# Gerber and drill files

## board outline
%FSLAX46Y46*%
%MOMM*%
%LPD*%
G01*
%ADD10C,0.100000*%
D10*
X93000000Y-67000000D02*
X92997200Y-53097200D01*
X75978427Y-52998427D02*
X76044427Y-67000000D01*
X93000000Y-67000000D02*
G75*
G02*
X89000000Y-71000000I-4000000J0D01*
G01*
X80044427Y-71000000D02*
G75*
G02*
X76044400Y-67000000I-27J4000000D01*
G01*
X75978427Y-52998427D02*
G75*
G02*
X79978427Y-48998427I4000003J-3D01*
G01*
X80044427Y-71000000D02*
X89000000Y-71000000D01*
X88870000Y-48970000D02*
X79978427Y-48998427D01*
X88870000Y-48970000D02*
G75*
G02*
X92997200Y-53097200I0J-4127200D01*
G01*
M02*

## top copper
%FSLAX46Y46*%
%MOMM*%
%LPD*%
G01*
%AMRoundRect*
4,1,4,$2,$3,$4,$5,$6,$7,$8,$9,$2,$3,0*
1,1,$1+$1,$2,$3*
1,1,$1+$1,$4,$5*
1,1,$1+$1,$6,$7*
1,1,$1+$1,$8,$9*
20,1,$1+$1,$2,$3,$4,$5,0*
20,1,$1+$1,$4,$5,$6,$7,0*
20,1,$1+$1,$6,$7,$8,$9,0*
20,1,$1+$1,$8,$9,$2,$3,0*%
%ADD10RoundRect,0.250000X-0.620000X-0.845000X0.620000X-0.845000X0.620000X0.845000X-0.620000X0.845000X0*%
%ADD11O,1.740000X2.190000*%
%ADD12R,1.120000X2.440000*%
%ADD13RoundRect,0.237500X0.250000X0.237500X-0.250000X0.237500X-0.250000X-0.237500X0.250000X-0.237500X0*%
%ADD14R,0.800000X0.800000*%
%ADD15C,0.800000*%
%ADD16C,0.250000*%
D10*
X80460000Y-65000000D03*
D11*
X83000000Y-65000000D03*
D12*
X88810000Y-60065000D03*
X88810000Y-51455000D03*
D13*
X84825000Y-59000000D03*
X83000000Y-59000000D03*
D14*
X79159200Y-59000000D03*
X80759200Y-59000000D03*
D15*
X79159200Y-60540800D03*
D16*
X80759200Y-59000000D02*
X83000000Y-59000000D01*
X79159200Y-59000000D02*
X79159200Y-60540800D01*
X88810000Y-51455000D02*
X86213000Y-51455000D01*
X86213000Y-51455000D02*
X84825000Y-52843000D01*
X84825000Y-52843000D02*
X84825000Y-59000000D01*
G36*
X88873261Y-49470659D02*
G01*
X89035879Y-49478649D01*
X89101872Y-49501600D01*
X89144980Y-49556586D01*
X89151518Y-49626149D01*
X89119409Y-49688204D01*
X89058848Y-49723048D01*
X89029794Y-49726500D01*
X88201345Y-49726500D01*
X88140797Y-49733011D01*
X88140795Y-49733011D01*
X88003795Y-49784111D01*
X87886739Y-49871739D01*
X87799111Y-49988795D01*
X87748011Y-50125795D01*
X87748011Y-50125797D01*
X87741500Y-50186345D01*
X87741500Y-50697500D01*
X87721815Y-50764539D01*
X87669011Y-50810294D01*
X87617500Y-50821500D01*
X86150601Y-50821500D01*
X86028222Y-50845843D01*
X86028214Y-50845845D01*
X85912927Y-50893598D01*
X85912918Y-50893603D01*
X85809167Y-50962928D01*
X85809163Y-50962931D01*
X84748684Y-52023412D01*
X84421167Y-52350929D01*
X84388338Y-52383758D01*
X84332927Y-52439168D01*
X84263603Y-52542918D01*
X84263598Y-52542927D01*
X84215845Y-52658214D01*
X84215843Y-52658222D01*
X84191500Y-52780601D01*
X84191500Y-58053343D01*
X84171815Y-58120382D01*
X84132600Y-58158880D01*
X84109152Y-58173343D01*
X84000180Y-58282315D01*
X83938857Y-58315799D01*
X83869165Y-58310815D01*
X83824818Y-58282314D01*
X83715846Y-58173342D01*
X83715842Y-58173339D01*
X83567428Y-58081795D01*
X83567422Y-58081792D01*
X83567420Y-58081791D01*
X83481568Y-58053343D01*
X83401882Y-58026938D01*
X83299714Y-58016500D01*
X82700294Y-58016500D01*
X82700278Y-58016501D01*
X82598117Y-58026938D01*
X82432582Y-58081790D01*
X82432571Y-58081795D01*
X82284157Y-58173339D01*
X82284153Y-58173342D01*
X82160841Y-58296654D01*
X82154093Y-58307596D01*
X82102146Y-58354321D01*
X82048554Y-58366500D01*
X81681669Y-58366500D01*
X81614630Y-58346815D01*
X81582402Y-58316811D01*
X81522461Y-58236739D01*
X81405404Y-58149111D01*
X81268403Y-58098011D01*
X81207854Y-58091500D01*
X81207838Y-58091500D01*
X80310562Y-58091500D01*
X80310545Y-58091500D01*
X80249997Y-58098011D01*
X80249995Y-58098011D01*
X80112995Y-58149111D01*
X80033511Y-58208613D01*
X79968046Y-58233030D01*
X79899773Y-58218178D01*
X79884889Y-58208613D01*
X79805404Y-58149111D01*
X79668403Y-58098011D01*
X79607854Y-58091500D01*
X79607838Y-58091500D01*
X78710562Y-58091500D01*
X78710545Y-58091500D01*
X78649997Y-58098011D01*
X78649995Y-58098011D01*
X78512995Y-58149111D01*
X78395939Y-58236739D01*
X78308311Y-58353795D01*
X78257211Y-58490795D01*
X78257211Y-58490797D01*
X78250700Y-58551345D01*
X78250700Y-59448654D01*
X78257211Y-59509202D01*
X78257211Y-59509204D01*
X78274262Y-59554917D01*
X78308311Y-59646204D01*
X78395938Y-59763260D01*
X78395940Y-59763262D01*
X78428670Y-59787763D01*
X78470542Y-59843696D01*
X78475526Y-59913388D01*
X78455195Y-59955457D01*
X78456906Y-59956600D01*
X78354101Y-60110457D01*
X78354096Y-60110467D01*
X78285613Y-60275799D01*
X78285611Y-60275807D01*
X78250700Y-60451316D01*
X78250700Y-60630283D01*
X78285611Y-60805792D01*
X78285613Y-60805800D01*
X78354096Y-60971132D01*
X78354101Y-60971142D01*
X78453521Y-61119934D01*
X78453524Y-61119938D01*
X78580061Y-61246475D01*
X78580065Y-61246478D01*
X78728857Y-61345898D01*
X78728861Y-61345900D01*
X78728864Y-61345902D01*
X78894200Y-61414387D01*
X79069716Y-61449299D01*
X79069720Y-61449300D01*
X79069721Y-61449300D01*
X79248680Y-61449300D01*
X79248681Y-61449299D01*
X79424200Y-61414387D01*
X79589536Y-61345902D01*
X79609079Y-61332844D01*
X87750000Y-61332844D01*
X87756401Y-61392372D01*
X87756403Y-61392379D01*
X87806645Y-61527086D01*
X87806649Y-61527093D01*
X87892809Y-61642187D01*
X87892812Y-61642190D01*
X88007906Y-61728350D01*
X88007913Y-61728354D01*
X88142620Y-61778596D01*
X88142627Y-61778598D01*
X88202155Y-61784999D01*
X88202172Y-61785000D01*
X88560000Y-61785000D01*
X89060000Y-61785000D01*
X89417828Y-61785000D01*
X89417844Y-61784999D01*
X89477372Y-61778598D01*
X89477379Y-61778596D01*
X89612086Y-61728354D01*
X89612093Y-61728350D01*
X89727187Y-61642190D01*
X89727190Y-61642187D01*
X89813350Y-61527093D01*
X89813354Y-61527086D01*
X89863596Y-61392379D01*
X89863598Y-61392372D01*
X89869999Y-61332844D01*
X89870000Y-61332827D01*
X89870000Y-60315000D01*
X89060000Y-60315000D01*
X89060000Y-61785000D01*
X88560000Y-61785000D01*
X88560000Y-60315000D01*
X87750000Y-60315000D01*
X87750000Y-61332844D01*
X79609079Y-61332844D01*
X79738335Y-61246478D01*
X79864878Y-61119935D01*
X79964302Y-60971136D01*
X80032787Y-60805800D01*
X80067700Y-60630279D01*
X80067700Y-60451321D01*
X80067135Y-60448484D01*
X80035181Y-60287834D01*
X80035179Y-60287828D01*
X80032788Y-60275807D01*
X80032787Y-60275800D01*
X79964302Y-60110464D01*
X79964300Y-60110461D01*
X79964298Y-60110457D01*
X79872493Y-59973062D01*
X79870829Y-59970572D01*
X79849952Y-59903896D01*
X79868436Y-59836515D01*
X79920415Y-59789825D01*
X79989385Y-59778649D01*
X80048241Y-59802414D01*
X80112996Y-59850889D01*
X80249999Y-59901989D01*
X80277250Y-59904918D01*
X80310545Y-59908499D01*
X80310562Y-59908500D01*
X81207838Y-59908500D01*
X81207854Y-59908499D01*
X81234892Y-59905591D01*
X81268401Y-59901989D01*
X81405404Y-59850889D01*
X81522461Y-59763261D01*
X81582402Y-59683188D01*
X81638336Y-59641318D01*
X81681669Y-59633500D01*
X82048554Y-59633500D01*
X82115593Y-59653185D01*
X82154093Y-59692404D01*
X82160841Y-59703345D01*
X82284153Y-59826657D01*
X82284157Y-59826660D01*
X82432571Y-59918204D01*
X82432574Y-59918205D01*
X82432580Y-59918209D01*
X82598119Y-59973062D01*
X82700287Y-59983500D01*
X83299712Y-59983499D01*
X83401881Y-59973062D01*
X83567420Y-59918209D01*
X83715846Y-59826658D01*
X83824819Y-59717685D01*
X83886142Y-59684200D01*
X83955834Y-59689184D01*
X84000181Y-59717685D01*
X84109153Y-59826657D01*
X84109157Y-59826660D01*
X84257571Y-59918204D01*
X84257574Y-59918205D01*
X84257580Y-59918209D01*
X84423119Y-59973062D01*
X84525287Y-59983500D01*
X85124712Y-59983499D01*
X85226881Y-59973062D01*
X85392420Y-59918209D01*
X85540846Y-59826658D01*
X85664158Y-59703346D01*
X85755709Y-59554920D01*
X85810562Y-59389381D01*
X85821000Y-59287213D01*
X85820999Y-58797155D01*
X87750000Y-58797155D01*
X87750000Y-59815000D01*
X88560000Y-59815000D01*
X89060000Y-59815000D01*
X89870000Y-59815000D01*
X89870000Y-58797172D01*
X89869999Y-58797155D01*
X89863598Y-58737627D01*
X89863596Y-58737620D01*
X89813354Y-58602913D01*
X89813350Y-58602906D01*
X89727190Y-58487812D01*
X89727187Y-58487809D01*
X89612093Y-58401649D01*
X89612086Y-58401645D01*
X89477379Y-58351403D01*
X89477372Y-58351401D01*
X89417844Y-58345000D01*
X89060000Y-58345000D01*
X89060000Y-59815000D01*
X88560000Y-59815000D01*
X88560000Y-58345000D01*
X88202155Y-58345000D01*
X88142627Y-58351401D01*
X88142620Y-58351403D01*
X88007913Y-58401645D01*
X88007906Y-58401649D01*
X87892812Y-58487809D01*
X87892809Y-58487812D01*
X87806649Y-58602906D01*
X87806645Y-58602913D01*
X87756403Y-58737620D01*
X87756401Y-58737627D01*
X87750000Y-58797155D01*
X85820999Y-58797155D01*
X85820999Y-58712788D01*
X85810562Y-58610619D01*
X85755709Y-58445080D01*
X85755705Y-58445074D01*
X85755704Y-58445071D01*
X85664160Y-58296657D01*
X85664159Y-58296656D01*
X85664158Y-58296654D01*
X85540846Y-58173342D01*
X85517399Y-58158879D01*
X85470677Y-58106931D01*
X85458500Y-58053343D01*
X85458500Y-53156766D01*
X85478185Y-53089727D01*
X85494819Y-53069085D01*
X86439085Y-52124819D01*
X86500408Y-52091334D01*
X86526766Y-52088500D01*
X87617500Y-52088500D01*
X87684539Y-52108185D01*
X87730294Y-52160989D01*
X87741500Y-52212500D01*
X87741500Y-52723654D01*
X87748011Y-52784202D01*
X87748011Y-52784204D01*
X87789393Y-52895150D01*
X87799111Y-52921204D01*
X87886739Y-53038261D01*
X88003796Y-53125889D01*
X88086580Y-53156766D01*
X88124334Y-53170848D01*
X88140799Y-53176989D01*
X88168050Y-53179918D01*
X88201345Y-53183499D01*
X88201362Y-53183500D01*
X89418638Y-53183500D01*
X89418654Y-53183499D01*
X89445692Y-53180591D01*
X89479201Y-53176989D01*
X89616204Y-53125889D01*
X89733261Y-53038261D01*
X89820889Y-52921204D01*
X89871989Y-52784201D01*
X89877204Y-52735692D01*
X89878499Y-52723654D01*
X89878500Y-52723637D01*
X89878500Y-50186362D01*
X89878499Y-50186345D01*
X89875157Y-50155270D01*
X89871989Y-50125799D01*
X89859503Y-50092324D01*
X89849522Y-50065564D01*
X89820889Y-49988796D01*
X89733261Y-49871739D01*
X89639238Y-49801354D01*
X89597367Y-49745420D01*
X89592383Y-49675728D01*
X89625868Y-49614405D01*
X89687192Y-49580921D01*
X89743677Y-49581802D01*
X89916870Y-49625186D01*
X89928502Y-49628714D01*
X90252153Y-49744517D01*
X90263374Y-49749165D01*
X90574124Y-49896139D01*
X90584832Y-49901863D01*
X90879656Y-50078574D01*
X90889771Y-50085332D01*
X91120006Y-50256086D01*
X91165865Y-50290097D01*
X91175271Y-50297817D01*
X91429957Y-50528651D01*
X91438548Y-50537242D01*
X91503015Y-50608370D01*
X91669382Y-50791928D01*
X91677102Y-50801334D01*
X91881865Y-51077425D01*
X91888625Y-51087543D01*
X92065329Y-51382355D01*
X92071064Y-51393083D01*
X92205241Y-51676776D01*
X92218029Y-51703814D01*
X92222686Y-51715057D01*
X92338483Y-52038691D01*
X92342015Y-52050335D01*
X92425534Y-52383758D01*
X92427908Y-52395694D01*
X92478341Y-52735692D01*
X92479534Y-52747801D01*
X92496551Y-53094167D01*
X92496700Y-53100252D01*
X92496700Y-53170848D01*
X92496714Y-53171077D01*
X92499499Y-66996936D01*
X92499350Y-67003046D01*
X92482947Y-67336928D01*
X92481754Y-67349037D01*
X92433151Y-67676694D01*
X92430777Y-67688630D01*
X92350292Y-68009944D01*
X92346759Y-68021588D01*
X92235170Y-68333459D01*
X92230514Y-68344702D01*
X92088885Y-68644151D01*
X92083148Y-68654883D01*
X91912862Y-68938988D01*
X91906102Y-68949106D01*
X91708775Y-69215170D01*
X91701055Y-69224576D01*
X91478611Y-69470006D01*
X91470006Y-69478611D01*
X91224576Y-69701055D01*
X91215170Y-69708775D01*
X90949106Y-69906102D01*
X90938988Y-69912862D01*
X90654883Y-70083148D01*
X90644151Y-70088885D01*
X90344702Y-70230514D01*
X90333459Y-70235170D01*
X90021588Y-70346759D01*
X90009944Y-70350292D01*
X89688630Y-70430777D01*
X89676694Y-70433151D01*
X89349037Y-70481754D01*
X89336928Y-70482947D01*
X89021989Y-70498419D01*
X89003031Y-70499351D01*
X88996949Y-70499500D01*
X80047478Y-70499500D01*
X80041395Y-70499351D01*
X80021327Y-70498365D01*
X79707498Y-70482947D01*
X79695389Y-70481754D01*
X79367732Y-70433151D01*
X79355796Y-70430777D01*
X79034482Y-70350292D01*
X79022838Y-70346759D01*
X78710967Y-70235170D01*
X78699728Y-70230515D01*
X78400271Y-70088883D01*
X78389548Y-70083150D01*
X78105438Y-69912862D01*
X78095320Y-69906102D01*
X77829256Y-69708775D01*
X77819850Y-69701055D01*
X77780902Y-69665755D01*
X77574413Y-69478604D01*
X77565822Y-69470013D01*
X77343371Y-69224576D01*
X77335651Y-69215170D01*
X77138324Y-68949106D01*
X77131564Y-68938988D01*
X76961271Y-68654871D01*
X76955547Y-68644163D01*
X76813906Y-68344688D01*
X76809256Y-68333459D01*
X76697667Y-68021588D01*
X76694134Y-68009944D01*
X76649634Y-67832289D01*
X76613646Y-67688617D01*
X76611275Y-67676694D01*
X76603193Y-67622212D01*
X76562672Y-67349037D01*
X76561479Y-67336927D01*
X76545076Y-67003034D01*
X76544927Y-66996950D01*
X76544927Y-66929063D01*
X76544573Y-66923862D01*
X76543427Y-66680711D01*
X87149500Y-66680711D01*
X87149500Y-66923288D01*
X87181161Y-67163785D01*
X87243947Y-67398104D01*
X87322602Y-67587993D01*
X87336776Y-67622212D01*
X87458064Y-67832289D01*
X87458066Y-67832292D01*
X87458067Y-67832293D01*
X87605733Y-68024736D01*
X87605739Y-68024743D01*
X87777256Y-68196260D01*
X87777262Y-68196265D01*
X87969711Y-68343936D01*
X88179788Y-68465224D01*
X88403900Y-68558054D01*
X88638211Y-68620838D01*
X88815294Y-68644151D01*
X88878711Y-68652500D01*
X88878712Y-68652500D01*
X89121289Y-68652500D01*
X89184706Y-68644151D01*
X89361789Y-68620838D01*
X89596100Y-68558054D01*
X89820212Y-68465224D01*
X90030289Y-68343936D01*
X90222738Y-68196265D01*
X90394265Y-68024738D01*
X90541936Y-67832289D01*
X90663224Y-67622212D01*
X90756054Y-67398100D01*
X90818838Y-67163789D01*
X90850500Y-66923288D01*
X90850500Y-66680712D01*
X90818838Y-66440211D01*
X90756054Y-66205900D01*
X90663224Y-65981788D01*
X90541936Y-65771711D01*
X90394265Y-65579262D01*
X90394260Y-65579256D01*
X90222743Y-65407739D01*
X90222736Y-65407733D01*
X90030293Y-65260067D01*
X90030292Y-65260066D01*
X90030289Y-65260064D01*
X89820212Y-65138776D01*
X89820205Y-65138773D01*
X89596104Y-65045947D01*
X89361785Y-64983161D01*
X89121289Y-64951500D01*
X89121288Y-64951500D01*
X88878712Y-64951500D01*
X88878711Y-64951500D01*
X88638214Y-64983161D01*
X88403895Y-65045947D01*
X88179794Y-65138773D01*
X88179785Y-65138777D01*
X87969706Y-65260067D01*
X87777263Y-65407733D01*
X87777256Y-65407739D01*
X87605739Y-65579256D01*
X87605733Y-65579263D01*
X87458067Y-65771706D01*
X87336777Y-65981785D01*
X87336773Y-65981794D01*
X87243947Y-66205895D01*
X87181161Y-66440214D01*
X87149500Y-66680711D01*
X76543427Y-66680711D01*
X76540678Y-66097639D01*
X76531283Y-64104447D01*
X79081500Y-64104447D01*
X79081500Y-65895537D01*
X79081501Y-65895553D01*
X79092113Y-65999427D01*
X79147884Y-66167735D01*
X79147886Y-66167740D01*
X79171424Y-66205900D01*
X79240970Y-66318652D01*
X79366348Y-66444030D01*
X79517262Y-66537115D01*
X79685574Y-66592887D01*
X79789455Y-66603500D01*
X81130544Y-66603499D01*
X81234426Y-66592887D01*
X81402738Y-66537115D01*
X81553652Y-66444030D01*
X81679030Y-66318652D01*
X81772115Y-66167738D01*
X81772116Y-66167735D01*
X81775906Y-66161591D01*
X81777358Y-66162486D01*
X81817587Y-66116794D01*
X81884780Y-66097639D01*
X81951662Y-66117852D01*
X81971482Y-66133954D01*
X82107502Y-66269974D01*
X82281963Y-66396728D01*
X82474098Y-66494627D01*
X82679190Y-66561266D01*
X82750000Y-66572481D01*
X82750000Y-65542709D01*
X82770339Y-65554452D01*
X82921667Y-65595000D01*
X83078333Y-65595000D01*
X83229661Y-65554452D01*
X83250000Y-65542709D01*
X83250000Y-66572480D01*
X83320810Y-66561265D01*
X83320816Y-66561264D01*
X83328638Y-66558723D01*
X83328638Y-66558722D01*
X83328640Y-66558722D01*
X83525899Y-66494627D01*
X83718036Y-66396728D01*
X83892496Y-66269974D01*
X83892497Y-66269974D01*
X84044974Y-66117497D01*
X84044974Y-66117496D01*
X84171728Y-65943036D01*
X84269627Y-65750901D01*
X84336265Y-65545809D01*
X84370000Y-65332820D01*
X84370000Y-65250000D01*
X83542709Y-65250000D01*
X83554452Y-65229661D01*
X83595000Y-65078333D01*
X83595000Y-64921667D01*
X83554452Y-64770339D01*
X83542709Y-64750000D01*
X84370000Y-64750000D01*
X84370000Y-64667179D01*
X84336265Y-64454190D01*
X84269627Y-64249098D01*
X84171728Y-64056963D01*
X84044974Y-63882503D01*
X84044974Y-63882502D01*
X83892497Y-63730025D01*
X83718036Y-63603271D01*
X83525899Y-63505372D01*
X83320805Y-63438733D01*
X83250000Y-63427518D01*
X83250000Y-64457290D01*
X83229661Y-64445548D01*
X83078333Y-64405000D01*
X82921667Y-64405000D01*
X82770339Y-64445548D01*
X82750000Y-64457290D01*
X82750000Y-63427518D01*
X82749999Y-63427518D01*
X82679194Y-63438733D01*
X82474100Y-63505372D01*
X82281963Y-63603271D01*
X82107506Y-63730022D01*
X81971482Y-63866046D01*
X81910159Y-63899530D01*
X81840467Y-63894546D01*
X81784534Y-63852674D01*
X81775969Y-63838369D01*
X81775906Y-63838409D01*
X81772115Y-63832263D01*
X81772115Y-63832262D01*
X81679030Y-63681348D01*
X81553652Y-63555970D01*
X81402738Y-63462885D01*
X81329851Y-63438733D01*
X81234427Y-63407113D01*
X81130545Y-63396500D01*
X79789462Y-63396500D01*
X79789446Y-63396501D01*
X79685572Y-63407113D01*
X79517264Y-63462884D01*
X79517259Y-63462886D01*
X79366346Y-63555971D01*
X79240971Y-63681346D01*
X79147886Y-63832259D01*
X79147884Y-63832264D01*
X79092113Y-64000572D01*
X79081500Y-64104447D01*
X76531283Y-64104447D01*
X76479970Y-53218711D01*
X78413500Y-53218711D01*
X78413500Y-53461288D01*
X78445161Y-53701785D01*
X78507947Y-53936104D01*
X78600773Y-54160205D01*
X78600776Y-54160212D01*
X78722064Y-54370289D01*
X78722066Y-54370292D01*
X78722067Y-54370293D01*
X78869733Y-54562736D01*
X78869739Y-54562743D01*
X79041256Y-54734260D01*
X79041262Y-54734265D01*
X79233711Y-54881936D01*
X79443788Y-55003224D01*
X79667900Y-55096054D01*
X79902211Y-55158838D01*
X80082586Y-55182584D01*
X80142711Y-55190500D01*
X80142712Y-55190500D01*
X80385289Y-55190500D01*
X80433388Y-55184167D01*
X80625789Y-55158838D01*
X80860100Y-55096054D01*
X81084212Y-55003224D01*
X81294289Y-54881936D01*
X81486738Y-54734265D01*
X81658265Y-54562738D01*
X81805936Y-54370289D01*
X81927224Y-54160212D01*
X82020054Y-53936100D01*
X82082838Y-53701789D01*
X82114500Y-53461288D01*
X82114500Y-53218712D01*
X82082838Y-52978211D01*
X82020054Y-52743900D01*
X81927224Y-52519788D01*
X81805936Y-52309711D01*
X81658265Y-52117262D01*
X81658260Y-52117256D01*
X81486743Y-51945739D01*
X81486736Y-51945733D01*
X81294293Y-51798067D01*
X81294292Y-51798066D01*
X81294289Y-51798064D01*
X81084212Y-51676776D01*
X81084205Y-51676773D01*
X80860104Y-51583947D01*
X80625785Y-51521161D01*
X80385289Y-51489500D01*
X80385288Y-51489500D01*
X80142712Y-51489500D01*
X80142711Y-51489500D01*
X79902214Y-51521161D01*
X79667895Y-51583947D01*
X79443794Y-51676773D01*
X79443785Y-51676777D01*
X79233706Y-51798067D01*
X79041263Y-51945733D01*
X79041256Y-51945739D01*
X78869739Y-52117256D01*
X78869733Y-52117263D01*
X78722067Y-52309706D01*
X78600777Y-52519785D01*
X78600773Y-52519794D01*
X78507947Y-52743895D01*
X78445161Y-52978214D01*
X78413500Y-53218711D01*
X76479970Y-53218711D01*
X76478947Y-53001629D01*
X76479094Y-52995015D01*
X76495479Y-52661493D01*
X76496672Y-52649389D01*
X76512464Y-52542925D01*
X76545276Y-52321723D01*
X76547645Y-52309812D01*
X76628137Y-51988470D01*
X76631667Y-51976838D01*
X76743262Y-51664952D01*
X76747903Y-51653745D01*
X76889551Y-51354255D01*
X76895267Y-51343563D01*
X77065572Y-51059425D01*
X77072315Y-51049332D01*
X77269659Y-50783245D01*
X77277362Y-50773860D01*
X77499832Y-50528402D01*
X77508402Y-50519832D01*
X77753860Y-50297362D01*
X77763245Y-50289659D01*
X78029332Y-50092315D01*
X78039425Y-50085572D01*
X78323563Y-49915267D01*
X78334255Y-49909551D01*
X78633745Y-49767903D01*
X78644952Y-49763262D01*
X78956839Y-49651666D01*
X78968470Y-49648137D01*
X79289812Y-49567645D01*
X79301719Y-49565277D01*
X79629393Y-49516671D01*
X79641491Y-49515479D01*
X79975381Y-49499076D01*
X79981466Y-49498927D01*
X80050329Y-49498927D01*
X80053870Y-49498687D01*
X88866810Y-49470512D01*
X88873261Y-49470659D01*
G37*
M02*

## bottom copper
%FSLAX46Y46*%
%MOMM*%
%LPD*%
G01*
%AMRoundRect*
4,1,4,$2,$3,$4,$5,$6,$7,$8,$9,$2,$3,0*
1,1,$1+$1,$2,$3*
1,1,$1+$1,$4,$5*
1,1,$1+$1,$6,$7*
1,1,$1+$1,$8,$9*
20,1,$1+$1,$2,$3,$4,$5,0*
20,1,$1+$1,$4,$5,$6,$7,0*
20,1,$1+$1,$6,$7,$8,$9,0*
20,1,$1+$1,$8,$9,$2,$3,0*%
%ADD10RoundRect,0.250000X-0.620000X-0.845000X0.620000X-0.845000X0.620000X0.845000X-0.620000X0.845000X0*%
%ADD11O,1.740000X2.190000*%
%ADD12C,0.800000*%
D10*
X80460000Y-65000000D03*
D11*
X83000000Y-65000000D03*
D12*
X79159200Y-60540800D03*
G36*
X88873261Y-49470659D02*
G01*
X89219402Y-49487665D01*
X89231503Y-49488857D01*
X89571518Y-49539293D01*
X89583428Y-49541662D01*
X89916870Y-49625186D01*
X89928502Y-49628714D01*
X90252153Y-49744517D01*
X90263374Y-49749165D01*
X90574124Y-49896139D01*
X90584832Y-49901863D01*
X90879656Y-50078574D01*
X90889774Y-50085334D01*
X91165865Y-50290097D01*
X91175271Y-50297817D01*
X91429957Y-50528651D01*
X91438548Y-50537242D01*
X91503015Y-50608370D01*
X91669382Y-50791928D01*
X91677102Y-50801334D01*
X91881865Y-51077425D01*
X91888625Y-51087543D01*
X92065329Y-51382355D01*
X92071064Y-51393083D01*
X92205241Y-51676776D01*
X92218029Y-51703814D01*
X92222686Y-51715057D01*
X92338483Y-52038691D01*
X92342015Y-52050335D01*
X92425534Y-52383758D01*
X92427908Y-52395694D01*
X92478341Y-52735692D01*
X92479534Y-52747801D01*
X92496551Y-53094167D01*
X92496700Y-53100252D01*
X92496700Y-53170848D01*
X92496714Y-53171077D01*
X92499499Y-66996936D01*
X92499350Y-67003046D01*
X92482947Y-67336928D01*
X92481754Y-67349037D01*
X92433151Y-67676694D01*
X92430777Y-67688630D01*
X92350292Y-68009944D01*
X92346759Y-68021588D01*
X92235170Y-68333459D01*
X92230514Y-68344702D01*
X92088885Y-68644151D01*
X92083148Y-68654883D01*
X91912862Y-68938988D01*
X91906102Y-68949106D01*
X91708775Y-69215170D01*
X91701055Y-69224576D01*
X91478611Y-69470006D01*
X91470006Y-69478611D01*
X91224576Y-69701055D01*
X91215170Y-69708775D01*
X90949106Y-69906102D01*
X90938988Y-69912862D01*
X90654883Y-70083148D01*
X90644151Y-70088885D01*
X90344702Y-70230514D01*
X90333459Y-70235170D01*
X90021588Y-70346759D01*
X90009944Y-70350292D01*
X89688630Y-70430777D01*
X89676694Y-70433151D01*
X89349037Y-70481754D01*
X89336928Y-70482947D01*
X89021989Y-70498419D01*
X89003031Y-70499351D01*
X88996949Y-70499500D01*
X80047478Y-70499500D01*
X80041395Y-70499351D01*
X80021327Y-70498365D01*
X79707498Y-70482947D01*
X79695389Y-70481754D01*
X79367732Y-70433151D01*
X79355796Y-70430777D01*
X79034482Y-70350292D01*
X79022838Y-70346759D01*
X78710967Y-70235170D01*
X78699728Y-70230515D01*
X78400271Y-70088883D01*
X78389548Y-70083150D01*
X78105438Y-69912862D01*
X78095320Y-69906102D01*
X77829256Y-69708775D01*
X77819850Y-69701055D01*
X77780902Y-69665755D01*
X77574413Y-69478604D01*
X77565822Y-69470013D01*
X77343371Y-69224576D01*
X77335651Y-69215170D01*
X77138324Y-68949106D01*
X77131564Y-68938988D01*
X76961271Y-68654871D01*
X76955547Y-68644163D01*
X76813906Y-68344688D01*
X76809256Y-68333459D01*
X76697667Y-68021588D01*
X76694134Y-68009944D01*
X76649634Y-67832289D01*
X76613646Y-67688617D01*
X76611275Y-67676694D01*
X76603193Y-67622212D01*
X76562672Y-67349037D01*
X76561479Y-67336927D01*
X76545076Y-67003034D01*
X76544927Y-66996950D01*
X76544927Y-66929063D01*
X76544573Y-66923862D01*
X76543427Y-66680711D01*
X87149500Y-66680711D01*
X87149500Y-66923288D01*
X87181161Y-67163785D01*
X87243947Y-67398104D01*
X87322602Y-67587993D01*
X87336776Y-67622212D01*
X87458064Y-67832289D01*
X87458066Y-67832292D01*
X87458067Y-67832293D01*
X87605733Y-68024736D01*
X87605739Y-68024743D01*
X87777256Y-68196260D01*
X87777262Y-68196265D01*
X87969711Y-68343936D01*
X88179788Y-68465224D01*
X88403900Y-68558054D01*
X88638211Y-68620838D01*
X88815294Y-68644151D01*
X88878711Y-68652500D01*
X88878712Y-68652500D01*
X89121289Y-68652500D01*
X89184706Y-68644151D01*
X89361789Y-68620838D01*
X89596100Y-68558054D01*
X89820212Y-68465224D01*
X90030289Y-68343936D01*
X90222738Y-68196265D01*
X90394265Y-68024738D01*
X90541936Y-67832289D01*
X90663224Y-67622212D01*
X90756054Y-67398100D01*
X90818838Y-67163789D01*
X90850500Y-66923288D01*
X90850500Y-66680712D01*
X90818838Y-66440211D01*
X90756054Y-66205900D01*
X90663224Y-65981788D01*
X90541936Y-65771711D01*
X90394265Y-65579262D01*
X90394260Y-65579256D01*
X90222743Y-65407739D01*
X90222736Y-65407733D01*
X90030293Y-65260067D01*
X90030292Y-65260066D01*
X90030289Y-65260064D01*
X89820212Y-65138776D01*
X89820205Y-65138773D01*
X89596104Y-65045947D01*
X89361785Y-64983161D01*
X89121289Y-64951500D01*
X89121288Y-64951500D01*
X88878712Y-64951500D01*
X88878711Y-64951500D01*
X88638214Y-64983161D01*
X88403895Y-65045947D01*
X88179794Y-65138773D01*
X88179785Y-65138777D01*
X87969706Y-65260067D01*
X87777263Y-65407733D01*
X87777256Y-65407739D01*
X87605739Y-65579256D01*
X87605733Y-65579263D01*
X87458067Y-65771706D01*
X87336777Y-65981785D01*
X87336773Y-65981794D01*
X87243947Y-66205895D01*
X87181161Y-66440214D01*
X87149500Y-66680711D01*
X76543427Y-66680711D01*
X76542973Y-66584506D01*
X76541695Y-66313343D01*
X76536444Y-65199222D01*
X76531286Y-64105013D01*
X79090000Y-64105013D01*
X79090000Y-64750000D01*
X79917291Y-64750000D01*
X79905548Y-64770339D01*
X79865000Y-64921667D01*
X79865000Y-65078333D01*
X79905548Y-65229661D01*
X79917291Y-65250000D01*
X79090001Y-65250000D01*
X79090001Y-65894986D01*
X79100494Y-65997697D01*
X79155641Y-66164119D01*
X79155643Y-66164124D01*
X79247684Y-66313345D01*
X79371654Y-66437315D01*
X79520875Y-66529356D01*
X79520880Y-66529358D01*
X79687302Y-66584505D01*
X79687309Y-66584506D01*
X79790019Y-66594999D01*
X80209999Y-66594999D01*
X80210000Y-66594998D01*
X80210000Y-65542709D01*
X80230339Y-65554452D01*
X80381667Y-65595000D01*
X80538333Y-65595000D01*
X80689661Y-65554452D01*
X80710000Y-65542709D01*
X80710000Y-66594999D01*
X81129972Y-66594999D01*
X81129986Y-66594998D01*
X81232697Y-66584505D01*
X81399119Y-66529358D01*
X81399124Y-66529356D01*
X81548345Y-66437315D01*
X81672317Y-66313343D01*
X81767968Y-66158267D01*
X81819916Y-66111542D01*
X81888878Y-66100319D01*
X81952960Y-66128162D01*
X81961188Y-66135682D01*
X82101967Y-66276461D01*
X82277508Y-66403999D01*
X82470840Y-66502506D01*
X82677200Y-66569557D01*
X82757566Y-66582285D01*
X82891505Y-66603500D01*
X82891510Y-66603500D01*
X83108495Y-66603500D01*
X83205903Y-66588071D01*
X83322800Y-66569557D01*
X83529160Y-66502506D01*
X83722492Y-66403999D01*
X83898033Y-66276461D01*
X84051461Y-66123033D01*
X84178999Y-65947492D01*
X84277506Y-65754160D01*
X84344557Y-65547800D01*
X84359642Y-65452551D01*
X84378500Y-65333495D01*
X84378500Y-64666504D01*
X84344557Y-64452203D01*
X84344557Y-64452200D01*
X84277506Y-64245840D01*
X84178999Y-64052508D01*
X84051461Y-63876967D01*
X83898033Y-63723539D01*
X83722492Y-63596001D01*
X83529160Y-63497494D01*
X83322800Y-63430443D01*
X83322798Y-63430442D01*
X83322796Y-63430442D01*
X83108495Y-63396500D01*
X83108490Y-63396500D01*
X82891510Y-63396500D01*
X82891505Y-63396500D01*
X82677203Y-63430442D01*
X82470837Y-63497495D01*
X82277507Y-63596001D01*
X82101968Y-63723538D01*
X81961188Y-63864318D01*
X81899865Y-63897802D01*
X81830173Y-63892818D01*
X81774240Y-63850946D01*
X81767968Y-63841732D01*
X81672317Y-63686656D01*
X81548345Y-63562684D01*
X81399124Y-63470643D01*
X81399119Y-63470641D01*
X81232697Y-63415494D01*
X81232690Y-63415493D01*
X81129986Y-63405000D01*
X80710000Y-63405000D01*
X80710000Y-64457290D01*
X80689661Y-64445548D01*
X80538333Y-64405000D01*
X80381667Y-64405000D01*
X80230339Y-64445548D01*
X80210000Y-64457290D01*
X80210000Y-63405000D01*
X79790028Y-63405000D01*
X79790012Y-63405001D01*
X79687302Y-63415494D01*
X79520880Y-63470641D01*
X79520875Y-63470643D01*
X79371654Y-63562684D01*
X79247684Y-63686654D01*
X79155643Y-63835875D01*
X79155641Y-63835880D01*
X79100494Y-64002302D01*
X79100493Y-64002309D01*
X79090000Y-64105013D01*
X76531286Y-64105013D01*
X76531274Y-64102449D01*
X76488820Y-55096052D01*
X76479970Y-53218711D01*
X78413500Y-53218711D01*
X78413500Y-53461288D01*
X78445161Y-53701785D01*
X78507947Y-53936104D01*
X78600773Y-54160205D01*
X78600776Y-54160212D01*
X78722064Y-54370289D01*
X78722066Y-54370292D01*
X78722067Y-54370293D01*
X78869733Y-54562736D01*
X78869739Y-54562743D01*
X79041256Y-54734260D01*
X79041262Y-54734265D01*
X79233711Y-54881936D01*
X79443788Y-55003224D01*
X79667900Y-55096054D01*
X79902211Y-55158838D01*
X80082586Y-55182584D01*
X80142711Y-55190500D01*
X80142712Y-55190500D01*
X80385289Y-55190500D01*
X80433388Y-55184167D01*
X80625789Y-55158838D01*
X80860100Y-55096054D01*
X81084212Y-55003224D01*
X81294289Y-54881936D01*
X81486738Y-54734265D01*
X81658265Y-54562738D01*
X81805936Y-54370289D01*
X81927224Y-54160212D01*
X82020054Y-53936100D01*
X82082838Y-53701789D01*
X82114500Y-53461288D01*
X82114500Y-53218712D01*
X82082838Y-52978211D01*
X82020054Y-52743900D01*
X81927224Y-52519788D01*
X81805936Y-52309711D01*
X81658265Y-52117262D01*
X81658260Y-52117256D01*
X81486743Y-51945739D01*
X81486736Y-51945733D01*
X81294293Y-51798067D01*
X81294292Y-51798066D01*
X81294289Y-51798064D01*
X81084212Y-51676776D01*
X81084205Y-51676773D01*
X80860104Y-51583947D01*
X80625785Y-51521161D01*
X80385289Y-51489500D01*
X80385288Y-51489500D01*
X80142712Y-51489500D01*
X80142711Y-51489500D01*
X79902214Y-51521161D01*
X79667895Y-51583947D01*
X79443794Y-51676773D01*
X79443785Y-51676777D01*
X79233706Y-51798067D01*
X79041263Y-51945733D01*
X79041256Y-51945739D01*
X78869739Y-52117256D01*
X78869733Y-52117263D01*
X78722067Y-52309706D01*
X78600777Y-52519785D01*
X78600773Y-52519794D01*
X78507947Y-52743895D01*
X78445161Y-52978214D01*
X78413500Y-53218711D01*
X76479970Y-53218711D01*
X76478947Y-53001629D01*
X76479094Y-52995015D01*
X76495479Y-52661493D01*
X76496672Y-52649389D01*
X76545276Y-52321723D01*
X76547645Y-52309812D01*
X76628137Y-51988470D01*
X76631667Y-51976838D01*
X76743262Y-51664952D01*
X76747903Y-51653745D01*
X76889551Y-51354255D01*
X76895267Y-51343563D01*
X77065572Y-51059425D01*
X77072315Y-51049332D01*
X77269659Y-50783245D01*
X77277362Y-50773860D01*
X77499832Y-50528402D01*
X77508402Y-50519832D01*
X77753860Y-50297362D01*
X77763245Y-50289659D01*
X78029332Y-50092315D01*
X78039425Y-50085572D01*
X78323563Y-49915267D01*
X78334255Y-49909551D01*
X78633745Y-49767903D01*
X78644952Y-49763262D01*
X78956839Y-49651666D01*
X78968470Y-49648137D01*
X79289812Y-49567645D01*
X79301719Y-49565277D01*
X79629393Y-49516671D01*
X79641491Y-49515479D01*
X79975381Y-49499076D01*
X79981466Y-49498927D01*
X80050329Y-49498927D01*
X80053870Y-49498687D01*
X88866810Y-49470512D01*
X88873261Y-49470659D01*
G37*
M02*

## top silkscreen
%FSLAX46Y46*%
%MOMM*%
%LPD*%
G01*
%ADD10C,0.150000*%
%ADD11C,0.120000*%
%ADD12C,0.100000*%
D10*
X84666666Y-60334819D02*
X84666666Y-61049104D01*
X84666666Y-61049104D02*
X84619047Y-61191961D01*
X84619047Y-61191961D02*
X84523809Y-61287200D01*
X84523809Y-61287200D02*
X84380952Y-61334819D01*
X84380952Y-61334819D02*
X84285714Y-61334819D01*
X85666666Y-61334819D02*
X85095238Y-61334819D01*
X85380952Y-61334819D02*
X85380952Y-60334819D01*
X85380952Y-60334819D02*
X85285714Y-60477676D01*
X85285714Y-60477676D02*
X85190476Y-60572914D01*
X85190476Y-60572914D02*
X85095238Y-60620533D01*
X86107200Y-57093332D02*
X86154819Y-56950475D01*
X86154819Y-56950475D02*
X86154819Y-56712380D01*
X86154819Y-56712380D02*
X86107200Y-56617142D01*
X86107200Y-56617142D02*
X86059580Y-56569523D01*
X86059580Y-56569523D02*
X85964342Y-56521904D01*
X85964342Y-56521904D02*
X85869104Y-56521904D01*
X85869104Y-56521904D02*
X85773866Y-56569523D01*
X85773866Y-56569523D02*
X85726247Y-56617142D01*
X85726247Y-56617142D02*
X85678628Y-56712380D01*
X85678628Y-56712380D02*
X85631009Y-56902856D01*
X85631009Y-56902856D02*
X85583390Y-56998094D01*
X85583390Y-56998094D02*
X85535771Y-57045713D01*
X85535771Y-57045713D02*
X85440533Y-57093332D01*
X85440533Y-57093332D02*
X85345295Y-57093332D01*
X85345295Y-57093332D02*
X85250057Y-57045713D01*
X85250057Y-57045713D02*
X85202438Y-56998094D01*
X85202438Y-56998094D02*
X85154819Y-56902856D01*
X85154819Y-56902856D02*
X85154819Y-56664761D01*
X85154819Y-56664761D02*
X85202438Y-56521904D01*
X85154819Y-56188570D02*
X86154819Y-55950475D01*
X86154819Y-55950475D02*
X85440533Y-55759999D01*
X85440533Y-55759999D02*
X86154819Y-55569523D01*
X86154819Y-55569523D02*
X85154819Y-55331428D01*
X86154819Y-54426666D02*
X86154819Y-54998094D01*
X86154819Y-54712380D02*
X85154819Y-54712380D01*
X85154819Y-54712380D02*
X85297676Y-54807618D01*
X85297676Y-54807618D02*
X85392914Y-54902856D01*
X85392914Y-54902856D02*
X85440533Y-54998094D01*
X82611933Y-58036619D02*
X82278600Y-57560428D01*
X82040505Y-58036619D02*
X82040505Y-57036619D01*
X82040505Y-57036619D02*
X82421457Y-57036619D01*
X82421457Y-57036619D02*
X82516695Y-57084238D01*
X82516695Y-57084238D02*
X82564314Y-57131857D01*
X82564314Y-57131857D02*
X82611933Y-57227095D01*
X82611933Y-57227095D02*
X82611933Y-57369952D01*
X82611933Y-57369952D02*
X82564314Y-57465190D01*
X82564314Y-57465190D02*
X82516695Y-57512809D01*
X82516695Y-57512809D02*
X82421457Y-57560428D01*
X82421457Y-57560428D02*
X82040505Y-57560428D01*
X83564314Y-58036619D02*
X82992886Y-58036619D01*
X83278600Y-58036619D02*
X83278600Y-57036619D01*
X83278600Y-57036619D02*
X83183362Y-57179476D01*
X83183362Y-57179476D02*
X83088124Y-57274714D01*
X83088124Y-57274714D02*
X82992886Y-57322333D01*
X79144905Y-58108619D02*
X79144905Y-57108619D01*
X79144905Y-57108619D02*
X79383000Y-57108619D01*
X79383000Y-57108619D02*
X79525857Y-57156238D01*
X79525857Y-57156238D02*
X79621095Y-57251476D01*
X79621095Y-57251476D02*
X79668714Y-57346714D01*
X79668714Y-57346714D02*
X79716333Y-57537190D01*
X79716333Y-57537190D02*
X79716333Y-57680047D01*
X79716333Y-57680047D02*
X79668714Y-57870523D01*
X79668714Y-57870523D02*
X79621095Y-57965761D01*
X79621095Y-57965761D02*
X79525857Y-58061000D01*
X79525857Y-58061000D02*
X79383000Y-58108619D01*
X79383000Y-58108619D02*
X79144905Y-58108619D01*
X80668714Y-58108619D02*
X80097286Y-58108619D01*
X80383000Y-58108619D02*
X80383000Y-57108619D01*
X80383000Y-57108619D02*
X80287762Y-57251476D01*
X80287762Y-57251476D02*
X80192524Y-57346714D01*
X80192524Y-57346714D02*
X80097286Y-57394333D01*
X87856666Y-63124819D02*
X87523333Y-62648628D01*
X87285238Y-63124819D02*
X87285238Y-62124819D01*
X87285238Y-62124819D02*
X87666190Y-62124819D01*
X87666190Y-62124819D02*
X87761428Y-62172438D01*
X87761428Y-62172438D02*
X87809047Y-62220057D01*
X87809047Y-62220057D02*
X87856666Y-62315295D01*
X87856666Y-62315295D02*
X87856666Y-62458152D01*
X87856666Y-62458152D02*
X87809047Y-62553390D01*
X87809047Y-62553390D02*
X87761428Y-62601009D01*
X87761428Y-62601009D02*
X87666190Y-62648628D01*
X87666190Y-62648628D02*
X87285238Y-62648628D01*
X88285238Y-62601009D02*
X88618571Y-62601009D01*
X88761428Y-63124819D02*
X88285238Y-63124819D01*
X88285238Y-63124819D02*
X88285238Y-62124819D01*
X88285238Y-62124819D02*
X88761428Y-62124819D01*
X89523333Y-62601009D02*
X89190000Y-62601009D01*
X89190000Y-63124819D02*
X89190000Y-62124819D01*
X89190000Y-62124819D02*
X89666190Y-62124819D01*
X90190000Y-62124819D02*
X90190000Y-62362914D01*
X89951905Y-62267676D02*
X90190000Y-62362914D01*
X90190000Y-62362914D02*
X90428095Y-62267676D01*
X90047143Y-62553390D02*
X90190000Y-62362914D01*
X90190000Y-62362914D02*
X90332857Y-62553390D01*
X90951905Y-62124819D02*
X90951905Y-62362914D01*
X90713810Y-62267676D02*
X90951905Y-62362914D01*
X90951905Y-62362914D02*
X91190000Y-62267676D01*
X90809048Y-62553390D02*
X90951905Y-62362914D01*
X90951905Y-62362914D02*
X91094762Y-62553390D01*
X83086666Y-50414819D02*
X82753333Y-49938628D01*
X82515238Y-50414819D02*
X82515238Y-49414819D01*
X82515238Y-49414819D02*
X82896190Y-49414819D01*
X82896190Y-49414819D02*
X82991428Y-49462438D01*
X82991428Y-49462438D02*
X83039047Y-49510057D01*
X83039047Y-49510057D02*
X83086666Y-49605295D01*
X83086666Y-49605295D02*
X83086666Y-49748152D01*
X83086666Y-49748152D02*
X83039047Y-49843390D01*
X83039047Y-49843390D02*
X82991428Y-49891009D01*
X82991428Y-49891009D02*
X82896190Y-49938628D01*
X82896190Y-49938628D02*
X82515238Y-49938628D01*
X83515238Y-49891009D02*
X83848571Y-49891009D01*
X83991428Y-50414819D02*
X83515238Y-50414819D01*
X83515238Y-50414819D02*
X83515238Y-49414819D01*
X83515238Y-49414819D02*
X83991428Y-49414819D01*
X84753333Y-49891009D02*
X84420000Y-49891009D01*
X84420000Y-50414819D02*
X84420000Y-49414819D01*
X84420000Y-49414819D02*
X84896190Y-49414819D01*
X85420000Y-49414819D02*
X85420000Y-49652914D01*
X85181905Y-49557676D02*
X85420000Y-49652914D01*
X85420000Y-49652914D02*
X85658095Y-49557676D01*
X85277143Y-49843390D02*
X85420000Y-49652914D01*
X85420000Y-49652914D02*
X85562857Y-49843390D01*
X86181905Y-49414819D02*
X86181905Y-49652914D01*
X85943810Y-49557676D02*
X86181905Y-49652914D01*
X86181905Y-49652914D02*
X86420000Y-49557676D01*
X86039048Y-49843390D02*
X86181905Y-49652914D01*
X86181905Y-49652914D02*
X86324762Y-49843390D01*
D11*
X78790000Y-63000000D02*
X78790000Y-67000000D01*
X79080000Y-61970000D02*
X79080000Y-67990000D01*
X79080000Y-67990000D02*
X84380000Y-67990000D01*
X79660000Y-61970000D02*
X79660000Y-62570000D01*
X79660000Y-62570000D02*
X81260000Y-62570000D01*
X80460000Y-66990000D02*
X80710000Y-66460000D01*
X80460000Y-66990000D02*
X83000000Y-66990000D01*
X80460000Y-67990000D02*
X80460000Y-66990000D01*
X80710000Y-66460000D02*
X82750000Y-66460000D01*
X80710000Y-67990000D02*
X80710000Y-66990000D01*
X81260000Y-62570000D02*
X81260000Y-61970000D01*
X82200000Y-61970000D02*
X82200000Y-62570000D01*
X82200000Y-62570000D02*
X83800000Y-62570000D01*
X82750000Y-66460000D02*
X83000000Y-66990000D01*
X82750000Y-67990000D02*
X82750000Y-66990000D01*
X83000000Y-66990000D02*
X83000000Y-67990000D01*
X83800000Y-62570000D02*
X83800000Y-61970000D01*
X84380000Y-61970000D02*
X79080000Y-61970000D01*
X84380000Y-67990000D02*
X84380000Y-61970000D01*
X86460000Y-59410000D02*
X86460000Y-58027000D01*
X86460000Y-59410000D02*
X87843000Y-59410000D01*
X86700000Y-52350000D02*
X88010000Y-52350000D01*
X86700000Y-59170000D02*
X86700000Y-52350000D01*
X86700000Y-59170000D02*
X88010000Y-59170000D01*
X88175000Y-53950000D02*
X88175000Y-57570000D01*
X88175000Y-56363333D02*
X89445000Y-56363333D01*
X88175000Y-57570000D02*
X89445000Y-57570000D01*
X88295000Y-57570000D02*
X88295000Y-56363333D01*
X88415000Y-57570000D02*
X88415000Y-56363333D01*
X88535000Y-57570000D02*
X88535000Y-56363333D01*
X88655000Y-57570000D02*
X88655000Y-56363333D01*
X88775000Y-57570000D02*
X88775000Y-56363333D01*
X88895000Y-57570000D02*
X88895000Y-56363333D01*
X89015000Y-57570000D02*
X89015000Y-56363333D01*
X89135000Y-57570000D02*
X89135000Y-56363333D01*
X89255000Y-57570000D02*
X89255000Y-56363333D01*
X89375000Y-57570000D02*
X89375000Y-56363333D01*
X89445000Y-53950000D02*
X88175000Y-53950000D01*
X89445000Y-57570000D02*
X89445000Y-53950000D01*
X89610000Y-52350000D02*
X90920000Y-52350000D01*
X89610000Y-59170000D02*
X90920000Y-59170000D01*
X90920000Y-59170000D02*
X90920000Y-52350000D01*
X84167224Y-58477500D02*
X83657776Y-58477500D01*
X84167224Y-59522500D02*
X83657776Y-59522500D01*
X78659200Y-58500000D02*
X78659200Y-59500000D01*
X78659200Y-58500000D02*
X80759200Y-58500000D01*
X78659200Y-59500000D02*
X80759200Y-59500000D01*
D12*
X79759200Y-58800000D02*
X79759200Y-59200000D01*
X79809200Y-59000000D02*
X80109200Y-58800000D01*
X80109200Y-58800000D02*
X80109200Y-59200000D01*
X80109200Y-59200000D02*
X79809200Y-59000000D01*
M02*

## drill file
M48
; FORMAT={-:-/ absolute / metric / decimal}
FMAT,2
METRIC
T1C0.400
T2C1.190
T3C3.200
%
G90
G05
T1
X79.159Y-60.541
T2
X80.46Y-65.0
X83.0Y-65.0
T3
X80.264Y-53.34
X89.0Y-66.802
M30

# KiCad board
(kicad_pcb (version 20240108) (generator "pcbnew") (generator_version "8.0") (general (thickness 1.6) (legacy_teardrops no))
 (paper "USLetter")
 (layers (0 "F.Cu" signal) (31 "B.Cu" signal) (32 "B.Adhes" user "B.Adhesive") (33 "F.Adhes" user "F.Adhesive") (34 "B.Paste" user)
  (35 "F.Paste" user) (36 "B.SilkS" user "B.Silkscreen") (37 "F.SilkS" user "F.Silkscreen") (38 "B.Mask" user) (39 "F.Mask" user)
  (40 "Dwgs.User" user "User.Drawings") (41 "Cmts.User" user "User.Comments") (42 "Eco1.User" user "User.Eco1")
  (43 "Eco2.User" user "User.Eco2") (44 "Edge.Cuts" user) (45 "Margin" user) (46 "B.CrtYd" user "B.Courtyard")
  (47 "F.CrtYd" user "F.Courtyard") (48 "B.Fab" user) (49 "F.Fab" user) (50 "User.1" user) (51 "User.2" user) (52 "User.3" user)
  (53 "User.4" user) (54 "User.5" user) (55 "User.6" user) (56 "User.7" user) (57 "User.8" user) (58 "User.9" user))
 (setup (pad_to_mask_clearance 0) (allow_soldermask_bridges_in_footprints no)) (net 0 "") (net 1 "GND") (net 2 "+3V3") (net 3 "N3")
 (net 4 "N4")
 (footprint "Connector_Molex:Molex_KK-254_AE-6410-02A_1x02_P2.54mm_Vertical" (layer "F.Cu") (at 80.46 65)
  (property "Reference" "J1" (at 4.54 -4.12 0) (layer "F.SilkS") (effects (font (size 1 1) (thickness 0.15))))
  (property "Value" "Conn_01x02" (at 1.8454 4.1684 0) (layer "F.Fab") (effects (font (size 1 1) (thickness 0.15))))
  (fp_line (start -1.67 -2) (end -1.67 2) (stroke (width 0.12) (type solid)) (layer "F.SilkS"))
  (fp_line (start -1.38 -3.03) (end -1.38 2.99) (stroke (width 0.12) (type solid)) (layer "F.SilkS"))
  (fp_line (start -1.38 2.99) (end 3.92 2.99) (stroke (width 0.12) (type solid)) (layer "F.SilkS"))
  (fp_line (start -0.8 -3.03) (end -0.8 -2.43) (stroke (width 0.12) (type solid)) (layer "F.SilkS"))
  (fp_line (start -0.8 -2.43) (end 0.8 -2.43) (stroke (width 0.12) (type solid)) (layer "F.SilkS"))
  (fp_line (start 0 1.99) (end 0.25 1.46) (stroke (width 0.12) (type solid)) (layer "F.SilkS"))
  (fp_line (start 0 1.99) (end 2.54 1.99) (stroke (width 0.12) (type solid)) (layer "F.SilkS"))
  (fp_line (start 0 2.99) (end 0 1.99) (stroke (width 0.12) (type solid)) (layer "F.SilkS"))
  (fp_line (start 0.25 1.46) (end 2.29 1.46) (stroke (width 0.12) (type solid)) (layer "F.SilkS"))
  (fp_line (start 0.25 2.99) (end 0.25 1.99) (stroke (width 0.12) (type solid)) (layer "F.SilkS"))
  (fp_line (start 0.8 -2.43) (end 0.8 -3.03) (stroke (width 0.12) (type solid)) (layer "F.SilkS"))
  (fp_line (start 1.74 -3.03) (end 1.74 -2.43) (stroke (width 0.12) (type solid)) (layer "F.SilkS"))
  (fp_line (start 1.74 -2.43) (end 3.34 -2.43) (stroke (width 0.12) (type solid)) (layer "F.SilkS"))
  (fp_line (start 2.29 1.46) (end 2.54 1.99) (stroke (width 0.12) (type solid)) (layer "F.SilkS"))
  (fp_line (start 2.29 2.99) (end 2.29 1.99) (stroke (width 0.12) (type solid)) (layer "F.SilkS"))
  (fp_line (start 2.54 1.99) (end 2.54 2.99) (stroke (width 0.12) (type solid)) (layer "F.SilkS"))
  (fp_line (start 3.34 -2.43) (end 3.34 -3.03) (stroke (width 0.12) (type solid)) (layer "F.SilkS"))
  (fp_line (start 3.92 -3.03) (end -1.38 -3.03) (stroke (width 0.12) (type solid)) (layer "F.SilkS"))
  (fp_line (start 3.92 2.99) (end 3.92 -3.03) (stroke (width 0.12) (type solid)) (layer "F.SilkS"))
  (pad "1" thru_hole roundrect (at 0 0) (size 1.74 2.19) (drill 1.19) (layers "*.Cu" "*.Mask") (remove_unused_layers no)
   (roundrect_rratio 0.143678) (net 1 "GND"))
  (pad "2" thru_hole oval (at 2.54 0) (size 1.74 2.19) (drill 1.19) (layers "*.Cu" "*.Mask") (remove_unused_layers no) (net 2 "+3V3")))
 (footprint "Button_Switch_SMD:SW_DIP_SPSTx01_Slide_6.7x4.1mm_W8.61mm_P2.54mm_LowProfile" (layer "F.Cu") (at 88.81 55.76 90)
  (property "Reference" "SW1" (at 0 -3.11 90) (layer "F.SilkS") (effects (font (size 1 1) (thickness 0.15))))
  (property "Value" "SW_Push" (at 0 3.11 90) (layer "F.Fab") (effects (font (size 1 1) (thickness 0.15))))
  (fp_line (start -3.65 -2.35) (end -2.267 -2.35) (stroke (width 0.12) (type solid)) (layer "F.SilkS"))
  (fp_line (start -3.65 -2.35) (end -3.65 -0.967) (stroke (width 0.12) (type solid)) (layer "F.SilkS"))
  (fp_line (start 3.41 -2.11) (end 3.41 -0.8) (stroke (width 0.12) (type solid)) (layer "F.SilkS"))
  (fp_line (start -3.41 -2.11) (end 3.41 -2.11) (stroke (width 0.12) (type solid)) (layer "F.SilkS"))
  (fp_line (start -3.41 -2.11) (end -3.41 -0.8) (stroke (width 0.12) (type solid)) (layer "F.SilkS"))
  (fp_line (start 1.81 -0.635) (end -1.81 -0.635) (stroke (width 0.12) (type solid)) (layer "F.SilkS"))
  (fp_line (start -0.603333 -0.635) (end -0.603333 0.635) (stroke (width 0.12) (type solid)) (layer "F.SilkS"))
  (fp_line (start -1.81 -0.635) (end -1.81 0.635) (stroke (width 0.12) (type solid)) (layer "F.SilkS"))
  (fp_line (start -1.81 -0.515) (end -0.603333 -0.515) (stroke (width 0.12) (type solid)) (layer "F.SilkS"))
  (fp_line (start -1.81 -0.395) (end -0.603333 -0.395) (stroke (width 0.12) (type solid)) (layer "F.SilkS"))
  (fp_line (start -1.81 -0.275) (end -0.603333 -0.275) (stroke (width 0.12) (type solid)) (layer "F.SilkS"))
  (fp_line (start -1.81 -0.155) (end -0.603333 -0.155) (stroke (width 0.12) (type solid)) (layer "F.SilkS"))
  (fp_line (start -1.81 -0.035) (end -0.603333 -0.035) (stroke (width 0.12) (type solid)) (layer "F.SilkS"))
  (fp_line (start -1.81 0.085) (end -0.603333 0.085) (stroke (width 0.12) (type solid)) (layer "F.SilkS"))
  (fp_line (start -1.81 0.205) (end -0.603333 0.205) (stroke (width 0.12) (type solid)) (layer "F.SilkS"))
  (fp_line (start -1.81 0.325) (end -0.603333 0.325) (stroke (width 0.12) (type solid)) (layer "F.SilkS"))
  (fp_line (start -1.81 0.445) (end -0.603333 0.445) (stroke (width 0.12) (type solid)) (layer "F.SilkS"))
  (fp_line (start -1.81 0.565) (end -0.603333 0.565) (stroke (width 0.12) (type solid)) (layer "F.SilkS"))
  (fp_line (start 1.81 0.635) (end 1.81 -0.635) (stroke (width 0.12) (type solid)) (layer "F.SilkS"))
  (fp_line (start -1.81 0.635) (end 1.81 0.635) (stroke (width 0.12) (type solid)) (layer "F.SilkS"))
  (fp_line (start 3.41 0.8) (end 3.41 2.11) (stroke (width 0.12) (type solid)) (layer "F.SilkS"))
  (fp_line (start -3.41 0.8) (end -3.41 2.11) (stroke (width 0.12) (type solid)) (layer "F.SilkS"))
  (fp_line (start -3.41 2.11) (end 3.41 2.11) (stroke (width 0.12) (type solid)) (layer "F.SilkS"))
  (pad "1" smd rect (at -4.305 0 90) (size 2.44 1.12) (layers "F.Cu" "F.Paste" "F.Mask") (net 2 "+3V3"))
  (pad "2" smd rect (at 4.305 0 90) (size 2.44 1.12) (layers "F.Cu" "F.Paste" "F.Mask") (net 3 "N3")))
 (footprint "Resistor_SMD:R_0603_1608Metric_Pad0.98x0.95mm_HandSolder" (layer "F.Cu") (at 83.9125 59 180)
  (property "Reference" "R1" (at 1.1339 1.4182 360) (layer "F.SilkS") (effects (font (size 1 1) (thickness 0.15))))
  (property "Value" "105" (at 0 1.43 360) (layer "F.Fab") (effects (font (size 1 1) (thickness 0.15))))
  (fp_line (start -0.254724 0.5225) (end 0.254724 0.5225) (stroke (width 0.12) (type solid)) (layer "F.SilkS"))
  (fp_line (start -0.254724 -0.5225) (end 0.254724 -0.5225) (stroke (width 0.12) (type solid)) (layer "F.SilkS"))
  (pad "1" smd roundrect (at -0.9125 0 180) (size 0.975 0.95) (layers "F.Cu" "F.Paste" "F.Mask") (roundrect_rratio 0.25) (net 3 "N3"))
  (pad "2" smd roundrect (at 0.9125 0 180) (size 0.975 0.95) (layers "F.Cu" "F.Paste" "F.Mask") (roundrect_rratio 0.25) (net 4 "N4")))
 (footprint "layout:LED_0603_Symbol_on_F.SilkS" (layer "F.Cu") (at 79.9592 59)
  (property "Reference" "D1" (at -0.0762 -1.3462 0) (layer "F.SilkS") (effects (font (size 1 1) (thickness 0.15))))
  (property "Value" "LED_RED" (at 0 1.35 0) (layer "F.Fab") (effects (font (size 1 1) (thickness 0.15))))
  (fp_line (start -1.3 -0.5) (end -1.3 0.5) (stroke (width 0.12) (type solid)) (layer "F.SilkS"))
  (fp_line (start -1.3 -0.5) (end 0.8 -0.5) (stroke (width 0.12) (type solid)) (layer "F.SilkS"))
  (fp_line (start -1.3 0.5) (end 0.8 0.5) (stroke (width 0.12) (type solid)) (layer "F.SilkS"))
  (fp_line (start -0.2 -0.2) (end -0.2 0.2) (stroke (width 0.1) (type solid)) (layer "F.SilkS"))
  (fp_line (start -0.15 0) (end 0.15 -0.2) (stroke (width 0.1) (type solid)) (layer "F.SilkS"))
  (fp_line (start 0.15 -0.2) (end 0.15 0.2) (stroke (width 0.1) (type solid)) (layer "F.SilkS"))
  (fp_line (start 0.15 0.2) (end -0.15 0) (stroke (width 0.1) (type solid)) (layer "F.SilkS"))
  (pad "1" smd rect (at -0.8 0 180) (size 0.8 0.8) (layers "F.Cu" "F.Paste" "F.Mask") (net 1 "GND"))
  (pad "2" smd rect (at 0.8 0 180) (size 0.8 0.8) (layers "F.Cu" "F.Paste" "F.Mask") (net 4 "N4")))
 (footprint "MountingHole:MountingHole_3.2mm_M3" (layer "F.Cu") (at 89 66.802)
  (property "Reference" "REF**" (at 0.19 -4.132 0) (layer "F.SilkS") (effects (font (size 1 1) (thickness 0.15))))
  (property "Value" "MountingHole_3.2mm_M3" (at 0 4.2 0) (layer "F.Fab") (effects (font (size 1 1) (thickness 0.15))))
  (pad "" np_thru_hole circle (at 0 0) (size 3.2 3.2) (drill 3.2) (layers "*.Cu" "*.Mask")))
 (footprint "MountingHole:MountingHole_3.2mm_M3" (layer "F.Cu") (at 80.264 53.34)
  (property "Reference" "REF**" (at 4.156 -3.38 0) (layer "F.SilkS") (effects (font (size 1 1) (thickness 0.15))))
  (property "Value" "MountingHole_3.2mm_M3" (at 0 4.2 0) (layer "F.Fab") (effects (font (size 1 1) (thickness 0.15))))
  (pad "" np_thru_hole circle (at 0 0) (size 3.2 3.2) (drill 3.2) (layers "*.Cu" "*.Mask")))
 (gr_line (start 93 67) (end 92.9972 53.0972) (stroke (width 0.1) (type default)) (layer "Edge.Cuts"))
 (gr_line (start 75.978427 52.998427) (end 76.044427 67) (stroke (width 0.1) (type default)) (layer "Edge.Cuts"))
 (gr_arc (start 93 67) (mid 91.828427 69.828427) (end 89 71) (stroke (width 0.1) (type default)) (layer "Edge.Cuts"))
 (gr_arc (start 80.044427 71) (mid 77.216 69.828427) (end 76.044427 67) (stroke (width 0.1) (type default)) (layer "Edge.Cuts"))
 (gr_arc (start 75.978427 52.998427) (mid 77.15 50.17) (end 79.978427 48.998427) (stroke (width 0.1) (type default)) (layer "Edge.Cuts"))
 (gr_line (start 80.044427 71) (end 89 71) (stroke (width 0.1) (type default)) (layer "Edge.Cuts"))
 (gr_line (start 88.87 48.97) (end 79.978427 48.998427) (stroke (width 0.1) (type default)) (layer "Edge.Cuts"))
 (gr_arc (start 88.87 48.97) (mid 91.788371 50.178829) (end 92.9972 53.0972) (stroke (width 0.1) (type default)) (layer "Edge.Cuts"))
 (segment (start 80.7592 59) (end 83 59) (width 0.25) (layer "F.Cu") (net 4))
 (segment (start 79.1592 59) (end 79.1592 60.5408) (width 0.25) (layer "F.Cu") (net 1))
 (via (at 79.1592 60.5408) (size 0.8) (drill 0.4) (layers "F.Cu" "B.Cu") (free yes) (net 1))
 (segment (start 88.81 51.455) (end 86.213 51.455) (width 0.25) (layer "F.Cu") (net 3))
 (segment (start 86.213 51.455) (end 84.825 52.843) (width 0.25) (layer "F.Cu") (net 3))
 (segment (start 84.825 52.843) (end 84.825 59) (width 0.25) (layer "F.Cu") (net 3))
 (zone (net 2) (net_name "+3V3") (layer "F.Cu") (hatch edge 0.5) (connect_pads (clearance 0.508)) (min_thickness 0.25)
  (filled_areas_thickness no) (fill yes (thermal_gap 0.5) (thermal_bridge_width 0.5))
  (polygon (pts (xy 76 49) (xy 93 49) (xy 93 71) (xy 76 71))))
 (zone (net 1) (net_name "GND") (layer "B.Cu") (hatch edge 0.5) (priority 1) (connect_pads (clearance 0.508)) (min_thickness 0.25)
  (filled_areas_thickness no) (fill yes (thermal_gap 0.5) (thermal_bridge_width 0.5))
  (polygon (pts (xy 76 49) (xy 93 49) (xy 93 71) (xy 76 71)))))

